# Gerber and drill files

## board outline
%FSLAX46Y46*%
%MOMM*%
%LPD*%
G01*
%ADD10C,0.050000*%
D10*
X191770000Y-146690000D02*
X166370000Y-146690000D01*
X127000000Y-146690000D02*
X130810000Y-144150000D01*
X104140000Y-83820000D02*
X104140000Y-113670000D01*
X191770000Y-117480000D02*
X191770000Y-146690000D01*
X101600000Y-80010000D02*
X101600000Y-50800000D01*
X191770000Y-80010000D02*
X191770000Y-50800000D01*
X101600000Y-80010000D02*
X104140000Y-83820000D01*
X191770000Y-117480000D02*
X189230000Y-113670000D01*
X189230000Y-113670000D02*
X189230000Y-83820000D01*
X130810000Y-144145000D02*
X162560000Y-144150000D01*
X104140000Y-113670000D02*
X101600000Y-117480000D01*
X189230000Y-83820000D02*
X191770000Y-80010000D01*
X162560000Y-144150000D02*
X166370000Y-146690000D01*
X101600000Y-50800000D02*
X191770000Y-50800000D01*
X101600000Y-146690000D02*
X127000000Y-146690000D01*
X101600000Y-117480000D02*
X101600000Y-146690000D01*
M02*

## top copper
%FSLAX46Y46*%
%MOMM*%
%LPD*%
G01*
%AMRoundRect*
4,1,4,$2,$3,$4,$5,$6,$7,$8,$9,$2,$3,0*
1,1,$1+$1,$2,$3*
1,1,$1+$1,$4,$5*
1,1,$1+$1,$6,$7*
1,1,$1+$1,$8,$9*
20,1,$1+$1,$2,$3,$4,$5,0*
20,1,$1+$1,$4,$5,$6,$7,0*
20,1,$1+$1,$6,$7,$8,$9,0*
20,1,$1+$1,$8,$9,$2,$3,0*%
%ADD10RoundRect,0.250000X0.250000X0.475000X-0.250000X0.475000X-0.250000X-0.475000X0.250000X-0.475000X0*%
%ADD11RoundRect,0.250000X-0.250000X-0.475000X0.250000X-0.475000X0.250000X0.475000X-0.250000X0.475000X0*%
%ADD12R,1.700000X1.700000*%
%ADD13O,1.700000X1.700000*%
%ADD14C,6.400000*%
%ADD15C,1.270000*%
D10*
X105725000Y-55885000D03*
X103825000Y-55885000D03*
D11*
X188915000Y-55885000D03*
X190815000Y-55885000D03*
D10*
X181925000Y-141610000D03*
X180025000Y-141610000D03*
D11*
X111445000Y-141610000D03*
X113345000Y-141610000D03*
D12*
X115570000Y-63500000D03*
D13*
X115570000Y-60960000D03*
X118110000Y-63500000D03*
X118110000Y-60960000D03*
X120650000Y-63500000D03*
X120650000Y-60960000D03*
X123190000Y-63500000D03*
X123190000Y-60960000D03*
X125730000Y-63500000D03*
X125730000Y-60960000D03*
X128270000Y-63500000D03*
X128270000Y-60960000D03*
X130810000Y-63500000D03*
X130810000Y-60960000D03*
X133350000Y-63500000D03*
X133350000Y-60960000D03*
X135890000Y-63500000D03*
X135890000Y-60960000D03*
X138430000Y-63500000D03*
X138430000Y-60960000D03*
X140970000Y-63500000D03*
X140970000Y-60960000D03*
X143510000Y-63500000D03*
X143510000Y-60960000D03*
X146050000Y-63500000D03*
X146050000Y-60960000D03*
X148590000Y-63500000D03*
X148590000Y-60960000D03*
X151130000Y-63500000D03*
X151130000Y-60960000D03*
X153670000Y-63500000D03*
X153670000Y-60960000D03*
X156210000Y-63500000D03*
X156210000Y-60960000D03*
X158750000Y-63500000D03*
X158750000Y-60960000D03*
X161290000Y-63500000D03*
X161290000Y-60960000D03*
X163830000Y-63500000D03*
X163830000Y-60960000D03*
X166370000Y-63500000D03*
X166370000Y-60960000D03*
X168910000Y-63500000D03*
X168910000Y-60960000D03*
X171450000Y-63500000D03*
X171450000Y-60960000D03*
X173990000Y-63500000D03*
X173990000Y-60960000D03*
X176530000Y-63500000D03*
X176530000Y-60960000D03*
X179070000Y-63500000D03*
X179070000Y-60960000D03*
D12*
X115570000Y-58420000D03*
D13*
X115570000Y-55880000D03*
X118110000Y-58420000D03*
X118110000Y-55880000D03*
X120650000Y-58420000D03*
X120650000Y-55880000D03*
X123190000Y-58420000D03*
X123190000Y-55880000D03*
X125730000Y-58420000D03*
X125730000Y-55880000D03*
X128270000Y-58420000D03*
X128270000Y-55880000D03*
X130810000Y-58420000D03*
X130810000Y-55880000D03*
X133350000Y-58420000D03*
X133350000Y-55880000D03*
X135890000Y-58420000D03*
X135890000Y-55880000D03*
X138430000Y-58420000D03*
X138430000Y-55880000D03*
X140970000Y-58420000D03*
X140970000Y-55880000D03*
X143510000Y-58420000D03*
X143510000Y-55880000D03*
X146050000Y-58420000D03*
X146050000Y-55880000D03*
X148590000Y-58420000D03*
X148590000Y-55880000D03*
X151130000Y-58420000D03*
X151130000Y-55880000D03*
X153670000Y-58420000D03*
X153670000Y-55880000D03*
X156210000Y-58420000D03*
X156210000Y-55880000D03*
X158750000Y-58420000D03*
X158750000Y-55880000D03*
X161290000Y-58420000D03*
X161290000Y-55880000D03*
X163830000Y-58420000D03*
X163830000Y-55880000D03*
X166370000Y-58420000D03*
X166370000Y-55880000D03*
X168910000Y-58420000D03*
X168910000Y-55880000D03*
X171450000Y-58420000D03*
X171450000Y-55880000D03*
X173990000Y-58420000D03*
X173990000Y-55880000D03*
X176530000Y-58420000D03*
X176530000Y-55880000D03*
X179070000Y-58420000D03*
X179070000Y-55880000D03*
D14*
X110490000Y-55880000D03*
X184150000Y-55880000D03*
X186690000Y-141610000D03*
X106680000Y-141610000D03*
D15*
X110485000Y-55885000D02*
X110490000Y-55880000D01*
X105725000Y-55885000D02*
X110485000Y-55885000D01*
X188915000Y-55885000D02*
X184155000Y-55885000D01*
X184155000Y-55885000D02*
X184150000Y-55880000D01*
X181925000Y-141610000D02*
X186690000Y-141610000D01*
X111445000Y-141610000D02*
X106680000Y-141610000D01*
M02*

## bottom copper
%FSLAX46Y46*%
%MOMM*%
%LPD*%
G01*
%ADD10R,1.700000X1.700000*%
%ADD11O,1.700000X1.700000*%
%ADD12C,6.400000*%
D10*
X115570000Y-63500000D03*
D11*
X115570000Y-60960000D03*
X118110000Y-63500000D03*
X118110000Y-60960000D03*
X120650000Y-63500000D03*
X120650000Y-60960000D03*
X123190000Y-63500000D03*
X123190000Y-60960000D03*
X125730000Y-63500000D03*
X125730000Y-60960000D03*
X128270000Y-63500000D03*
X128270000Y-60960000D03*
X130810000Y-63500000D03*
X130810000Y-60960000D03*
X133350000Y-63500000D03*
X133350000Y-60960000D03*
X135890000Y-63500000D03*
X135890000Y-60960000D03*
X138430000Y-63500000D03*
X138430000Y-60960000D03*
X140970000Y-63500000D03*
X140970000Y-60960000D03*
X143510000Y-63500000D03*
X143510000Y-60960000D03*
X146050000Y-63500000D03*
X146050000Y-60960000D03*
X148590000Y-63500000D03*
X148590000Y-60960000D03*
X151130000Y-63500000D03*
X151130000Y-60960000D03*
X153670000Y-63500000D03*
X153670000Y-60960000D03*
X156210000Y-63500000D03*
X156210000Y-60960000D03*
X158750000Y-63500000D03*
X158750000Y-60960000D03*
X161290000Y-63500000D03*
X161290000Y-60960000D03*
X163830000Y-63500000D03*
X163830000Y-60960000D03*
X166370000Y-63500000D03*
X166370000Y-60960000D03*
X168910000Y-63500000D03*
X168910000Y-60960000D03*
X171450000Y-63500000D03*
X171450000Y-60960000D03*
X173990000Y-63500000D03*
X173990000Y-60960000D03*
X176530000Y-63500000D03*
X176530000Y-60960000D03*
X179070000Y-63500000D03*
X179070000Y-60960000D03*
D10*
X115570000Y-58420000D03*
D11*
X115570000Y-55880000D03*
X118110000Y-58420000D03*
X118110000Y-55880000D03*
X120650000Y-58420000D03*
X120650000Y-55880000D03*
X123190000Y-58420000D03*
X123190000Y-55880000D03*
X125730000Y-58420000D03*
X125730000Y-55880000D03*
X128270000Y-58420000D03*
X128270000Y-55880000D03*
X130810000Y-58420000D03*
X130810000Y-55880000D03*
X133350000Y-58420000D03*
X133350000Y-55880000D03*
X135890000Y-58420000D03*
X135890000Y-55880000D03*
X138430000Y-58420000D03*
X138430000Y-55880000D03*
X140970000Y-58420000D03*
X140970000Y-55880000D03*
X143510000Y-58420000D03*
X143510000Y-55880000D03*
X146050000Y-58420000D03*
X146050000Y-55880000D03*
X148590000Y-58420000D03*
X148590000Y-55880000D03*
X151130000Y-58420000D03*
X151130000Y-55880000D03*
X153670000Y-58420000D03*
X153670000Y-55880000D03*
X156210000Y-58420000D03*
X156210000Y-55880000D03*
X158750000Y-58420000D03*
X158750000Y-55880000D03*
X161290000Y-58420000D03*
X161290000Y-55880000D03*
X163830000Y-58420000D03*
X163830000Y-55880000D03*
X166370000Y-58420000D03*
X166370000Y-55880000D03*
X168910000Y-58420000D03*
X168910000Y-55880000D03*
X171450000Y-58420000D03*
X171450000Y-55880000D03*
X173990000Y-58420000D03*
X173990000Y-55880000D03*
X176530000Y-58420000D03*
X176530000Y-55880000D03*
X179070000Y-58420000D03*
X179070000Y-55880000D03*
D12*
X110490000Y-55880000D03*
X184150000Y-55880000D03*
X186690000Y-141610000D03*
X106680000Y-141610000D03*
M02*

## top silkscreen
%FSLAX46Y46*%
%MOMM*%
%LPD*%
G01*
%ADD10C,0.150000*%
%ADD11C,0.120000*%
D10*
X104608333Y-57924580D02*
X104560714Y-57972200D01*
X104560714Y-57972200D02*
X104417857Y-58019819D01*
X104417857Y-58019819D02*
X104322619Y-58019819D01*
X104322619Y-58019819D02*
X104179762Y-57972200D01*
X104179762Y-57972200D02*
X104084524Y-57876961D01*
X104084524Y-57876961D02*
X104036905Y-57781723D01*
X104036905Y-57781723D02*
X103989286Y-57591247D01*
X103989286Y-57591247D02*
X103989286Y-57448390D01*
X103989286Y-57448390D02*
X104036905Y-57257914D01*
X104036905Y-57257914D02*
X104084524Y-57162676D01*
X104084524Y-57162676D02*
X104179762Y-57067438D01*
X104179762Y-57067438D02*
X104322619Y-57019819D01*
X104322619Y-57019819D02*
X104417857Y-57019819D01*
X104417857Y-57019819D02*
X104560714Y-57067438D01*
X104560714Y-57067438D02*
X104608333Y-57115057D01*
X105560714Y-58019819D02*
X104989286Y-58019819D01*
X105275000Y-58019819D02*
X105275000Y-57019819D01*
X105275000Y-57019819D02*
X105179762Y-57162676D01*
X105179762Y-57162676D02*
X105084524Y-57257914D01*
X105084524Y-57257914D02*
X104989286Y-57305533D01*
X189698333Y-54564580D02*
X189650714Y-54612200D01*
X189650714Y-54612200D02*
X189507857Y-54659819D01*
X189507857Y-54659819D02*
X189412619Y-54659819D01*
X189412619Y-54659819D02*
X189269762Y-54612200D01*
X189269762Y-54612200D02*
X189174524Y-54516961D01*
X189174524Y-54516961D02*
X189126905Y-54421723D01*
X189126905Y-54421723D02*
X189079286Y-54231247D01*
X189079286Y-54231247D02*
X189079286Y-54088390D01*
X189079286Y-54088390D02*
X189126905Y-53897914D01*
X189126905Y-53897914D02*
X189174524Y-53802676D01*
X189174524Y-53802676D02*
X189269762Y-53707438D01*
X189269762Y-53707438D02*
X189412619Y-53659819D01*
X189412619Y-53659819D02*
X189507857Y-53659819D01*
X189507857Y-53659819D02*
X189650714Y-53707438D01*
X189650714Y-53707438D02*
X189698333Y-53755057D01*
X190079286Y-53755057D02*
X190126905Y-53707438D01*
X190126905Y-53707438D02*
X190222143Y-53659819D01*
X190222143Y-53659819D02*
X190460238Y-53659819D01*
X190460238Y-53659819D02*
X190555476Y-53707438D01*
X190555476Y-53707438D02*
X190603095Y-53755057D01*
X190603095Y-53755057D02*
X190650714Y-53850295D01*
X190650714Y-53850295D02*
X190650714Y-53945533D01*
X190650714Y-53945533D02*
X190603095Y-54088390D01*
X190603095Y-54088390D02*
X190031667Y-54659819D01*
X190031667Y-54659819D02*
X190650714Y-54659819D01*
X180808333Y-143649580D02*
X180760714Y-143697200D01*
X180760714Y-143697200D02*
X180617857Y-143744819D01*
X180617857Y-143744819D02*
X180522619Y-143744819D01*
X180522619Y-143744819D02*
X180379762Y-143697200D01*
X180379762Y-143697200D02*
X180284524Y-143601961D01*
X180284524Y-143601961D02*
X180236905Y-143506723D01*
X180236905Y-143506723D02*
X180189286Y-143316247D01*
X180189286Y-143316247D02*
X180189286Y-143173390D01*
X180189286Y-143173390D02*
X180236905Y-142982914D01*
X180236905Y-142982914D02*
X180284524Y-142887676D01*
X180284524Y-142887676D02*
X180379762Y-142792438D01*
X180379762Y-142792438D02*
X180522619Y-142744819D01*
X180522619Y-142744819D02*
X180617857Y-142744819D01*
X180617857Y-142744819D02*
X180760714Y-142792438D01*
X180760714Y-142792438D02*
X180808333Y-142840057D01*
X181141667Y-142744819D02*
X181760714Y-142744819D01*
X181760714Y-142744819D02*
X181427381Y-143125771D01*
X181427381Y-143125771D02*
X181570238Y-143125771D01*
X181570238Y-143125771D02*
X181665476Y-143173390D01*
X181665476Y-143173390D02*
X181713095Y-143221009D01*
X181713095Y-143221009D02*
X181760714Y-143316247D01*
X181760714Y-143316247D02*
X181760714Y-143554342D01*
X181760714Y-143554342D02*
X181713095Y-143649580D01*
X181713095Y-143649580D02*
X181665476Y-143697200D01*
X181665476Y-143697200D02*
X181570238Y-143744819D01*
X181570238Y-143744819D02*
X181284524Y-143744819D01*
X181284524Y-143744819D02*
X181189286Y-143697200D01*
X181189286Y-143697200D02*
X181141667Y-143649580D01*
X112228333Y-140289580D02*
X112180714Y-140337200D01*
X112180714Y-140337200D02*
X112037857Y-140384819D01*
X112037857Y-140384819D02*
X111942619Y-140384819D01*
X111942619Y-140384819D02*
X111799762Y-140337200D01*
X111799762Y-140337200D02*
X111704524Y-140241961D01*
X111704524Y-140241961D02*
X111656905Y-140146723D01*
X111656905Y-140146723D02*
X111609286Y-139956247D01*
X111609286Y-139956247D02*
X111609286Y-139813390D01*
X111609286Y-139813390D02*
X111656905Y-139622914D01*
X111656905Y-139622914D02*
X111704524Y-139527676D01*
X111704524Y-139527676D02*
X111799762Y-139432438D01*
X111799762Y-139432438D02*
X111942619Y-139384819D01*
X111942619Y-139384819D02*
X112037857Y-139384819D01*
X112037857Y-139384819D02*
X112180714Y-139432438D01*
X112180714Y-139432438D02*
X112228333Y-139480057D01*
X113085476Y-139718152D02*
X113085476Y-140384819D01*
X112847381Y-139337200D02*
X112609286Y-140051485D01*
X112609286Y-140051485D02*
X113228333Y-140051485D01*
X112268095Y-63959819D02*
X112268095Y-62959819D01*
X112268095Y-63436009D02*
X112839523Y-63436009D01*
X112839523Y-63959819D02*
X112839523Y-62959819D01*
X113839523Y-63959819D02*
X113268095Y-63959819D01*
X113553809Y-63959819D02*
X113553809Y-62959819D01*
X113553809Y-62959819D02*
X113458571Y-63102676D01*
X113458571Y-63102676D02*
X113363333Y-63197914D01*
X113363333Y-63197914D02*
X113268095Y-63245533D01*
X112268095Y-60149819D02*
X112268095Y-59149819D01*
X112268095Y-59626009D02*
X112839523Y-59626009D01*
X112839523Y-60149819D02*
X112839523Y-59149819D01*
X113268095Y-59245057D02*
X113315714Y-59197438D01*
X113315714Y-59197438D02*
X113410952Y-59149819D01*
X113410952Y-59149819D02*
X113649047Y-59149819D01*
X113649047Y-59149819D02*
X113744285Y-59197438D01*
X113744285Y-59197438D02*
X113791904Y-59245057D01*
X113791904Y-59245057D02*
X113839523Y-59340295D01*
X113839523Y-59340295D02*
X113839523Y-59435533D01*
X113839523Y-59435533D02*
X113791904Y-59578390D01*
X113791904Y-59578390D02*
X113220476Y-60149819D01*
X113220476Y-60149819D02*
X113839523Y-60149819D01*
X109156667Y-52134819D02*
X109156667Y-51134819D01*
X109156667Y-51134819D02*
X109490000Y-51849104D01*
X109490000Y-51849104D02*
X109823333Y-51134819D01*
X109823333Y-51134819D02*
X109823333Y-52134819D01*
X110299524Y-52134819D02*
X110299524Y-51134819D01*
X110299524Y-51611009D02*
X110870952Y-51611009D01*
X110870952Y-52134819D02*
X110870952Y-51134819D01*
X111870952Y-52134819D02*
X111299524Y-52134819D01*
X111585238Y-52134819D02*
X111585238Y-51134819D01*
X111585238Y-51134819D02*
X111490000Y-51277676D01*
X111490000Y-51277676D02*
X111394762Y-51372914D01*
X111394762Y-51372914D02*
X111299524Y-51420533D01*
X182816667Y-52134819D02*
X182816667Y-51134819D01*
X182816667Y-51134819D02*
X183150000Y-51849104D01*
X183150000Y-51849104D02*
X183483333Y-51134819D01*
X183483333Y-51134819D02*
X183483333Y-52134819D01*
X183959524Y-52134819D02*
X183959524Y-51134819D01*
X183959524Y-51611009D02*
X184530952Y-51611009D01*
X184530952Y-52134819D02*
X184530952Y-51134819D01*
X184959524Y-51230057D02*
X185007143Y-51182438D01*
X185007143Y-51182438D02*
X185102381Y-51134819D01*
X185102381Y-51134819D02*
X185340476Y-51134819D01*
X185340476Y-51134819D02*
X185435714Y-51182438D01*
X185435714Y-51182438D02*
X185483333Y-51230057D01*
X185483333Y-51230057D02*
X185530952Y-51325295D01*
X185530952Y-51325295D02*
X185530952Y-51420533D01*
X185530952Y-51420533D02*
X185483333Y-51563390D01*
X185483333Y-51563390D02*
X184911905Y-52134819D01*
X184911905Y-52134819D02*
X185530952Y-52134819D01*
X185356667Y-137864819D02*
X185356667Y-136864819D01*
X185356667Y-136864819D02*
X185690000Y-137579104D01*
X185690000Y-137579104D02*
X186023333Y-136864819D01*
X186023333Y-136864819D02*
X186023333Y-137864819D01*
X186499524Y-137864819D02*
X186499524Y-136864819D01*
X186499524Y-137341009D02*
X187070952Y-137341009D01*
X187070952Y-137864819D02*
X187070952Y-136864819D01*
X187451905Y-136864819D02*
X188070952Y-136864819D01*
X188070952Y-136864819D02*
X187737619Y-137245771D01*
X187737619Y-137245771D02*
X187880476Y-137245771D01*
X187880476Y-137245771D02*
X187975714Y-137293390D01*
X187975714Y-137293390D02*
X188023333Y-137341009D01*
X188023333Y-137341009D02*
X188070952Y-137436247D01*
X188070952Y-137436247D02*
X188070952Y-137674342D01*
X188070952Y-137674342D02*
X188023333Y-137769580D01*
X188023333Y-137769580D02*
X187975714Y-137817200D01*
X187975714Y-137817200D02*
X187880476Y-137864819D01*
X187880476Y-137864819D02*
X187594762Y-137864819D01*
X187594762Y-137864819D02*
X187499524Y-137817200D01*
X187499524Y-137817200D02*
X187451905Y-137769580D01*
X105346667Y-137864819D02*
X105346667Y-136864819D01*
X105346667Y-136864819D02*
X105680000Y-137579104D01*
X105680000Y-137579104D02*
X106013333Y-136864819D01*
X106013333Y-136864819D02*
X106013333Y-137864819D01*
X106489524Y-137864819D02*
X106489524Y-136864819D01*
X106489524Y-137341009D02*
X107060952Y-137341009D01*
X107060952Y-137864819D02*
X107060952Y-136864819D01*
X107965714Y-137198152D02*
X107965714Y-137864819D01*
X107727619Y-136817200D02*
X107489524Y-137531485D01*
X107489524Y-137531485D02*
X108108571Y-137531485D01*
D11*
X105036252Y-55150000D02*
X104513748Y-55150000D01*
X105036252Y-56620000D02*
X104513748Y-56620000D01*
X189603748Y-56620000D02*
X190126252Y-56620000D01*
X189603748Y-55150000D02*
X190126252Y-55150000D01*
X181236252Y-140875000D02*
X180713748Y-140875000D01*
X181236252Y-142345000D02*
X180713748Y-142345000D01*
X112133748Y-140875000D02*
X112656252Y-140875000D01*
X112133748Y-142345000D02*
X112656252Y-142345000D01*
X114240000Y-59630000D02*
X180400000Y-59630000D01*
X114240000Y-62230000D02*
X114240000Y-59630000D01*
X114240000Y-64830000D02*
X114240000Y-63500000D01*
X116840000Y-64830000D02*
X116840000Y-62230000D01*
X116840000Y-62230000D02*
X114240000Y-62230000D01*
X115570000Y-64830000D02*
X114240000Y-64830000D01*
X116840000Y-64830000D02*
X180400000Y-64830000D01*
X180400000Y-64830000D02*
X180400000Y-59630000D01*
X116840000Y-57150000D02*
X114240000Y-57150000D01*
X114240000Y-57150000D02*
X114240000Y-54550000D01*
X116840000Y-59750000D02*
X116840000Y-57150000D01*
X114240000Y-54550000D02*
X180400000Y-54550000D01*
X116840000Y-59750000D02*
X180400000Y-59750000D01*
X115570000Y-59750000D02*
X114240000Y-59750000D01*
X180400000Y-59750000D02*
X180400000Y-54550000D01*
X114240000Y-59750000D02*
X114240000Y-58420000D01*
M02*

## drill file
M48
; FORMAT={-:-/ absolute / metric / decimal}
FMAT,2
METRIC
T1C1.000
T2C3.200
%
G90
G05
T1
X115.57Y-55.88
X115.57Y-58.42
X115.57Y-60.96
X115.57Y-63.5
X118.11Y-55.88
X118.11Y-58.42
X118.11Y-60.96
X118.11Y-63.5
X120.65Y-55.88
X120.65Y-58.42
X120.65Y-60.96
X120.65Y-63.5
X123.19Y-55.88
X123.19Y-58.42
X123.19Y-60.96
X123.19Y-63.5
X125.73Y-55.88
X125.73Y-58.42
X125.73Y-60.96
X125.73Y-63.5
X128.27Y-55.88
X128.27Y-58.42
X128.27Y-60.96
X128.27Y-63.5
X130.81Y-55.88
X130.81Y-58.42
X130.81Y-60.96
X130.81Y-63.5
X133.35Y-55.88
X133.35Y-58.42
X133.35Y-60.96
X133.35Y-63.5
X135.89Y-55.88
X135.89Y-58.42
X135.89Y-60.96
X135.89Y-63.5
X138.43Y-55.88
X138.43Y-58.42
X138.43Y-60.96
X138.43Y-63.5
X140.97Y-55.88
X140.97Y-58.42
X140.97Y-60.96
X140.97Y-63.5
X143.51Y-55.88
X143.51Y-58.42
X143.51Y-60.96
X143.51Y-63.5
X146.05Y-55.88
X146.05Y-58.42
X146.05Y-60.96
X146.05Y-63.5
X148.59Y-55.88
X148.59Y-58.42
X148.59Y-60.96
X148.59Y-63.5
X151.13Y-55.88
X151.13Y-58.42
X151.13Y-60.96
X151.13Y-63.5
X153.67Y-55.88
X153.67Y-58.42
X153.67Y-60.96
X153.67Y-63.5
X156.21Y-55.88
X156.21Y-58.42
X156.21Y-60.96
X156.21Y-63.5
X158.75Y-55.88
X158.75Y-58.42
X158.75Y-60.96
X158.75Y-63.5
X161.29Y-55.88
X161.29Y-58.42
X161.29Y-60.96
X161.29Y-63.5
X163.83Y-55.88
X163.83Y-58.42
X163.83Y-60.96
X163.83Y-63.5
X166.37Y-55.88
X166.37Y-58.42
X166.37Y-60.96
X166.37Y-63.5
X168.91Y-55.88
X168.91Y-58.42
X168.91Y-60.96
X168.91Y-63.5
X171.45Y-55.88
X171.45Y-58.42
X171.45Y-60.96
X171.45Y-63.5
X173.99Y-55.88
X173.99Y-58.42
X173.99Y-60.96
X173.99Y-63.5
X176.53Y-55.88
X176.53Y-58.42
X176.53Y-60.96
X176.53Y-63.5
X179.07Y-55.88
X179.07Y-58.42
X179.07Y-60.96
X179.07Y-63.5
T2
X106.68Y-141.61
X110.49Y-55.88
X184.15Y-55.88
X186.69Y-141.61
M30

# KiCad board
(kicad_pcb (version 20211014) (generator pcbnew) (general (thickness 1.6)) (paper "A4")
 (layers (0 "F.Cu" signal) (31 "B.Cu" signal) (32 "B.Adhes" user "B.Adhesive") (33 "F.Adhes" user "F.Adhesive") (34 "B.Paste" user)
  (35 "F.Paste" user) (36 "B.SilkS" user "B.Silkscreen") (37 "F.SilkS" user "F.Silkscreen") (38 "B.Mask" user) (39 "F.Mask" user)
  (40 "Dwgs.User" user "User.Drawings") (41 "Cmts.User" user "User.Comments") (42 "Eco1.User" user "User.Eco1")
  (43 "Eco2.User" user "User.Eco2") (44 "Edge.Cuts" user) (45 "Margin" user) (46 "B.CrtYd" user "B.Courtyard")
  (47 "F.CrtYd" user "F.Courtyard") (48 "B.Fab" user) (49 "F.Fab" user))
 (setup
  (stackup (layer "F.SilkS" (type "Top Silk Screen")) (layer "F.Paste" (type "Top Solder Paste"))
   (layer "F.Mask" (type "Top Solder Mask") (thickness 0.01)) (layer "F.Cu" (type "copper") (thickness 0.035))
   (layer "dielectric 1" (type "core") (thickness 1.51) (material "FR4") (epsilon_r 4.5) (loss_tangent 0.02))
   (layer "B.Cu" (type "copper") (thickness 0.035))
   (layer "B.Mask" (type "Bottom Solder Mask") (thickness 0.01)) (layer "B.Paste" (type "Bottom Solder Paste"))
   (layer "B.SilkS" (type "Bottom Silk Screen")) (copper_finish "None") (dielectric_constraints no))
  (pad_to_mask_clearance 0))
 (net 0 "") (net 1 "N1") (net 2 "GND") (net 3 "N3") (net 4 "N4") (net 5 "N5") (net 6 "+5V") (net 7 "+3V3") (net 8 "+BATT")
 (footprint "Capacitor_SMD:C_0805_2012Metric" (layer "F.Cu") (at 104.775 55.885 180)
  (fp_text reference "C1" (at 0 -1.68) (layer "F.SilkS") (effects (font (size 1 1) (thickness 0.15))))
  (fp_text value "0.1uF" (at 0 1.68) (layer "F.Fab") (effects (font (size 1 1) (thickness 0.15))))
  (fp_line (start -0.261252 0.735) (end 0.261252 0.735) (layer "F.SilkS") (width 0.12))
  (fp_line (start -0.261252 -0.735) (end 0.261252 -0.735) (layer "F.SilkS") (width 0.12))
  (pad "1" smd roundrect locked (at -0.95 0 180) (size 1 1.45) (layers "F.Cu" "F.Paste" "F.Mask") (roundrect_rratio 0.25) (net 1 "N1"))
  (pad "2" smd roundrect locked (at 0.95 0 180) (size 1 1.45) (layers "F.Cu" "F.Paste" "F.Mask") (roundrect_rratio 0.25) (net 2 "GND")))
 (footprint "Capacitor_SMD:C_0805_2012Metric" (layer "F.Cu") (at 189.865 55.885)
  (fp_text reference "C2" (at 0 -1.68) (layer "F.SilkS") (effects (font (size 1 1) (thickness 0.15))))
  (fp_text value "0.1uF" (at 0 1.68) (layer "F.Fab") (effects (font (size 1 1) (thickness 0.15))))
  (fp_line (start -0.261252 0.735) (end 0.261252 0.735) (layer "F.SilkS") (width 0.12))
  (fp_line (start -0.261252 -0.735) (end 0.261252 -0.735) (layer "F.SilkS") (width 0.12))
  (pad "1" smd roundrect locked (at -0.95 0) (size 1 1.45) (layers "F.Cu" "F.Paste" "F.Mask") (roundrect_rratio 0.25) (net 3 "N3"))
  (pad "2" smd roundrect locked (at 0.95 0) (size 1 1.45) (layers "F.Cu" "F.Paste" "F.Mask") (roundrect_rratio 0.25) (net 2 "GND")))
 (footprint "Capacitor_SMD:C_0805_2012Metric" (layer "F.Cu") (at 180.975 141.61 180)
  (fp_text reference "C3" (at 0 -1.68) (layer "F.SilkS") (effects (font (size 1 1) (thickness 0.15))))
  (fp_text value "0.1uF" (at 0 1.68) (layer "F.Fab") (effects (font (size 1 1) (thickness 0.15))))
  (fp_line (start -0.261252 0.735) (end 0.261252 0.735) (layer "F.SilkS") (width 0.12))
  (fp_line (start -0.261252 -0.735) (end 0.261252 -0.735) (layer "F.SilkS") (width 0.12))
  (pad "1" smd roundrect locked (at -0.95 0 180) (size 1 1.45) (layers "F.Cu" "F.Paste" "F.Mask") (roundrect_rratio 0.25) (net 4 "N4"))
  (pad "2" smd roundrect locked (at 0.95 0 180) (size 1 1.45) (layers "F.Cu" "F.Paste" "F.Mask") (roundrect_rratio 0.25) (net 2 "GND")))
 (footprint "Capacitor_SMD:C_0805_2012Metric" (layer "F.Cu") (at 112.395 141.61)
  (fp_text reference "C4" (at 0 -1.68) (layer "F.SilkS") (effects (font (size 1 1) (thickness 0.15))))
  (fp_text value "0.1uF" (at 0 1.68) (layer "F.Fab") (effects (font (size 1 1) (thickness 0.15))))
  (fp_line (start -0.261252 -0.735) (end 0.261252 -0.735) (layer "F.SilkS") (width 0.12))
  (fp_line (start -0.261252 0.735) (end 0.261252 0.735) (layer "F.SilkS") (width 0.12))
  (pad "1" smd roundrect locked (at -0.95 0) (size 1 1.45) (layers "F.Cu" "F.Paste" "F.Mask") (roundrect_rratio 0.25) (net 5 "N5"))
  (pad "2" smd roundrect locked (at 0.95 0) (size 1 1.45) (layers "F.Cu" "F.Paste" "F.Mask") (roundrect_rratio 0.25) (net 2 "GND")))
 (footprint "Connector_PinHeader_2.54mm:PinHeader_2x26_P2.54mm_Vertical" (layer "F.Cu") (at 115.57 63.5 90)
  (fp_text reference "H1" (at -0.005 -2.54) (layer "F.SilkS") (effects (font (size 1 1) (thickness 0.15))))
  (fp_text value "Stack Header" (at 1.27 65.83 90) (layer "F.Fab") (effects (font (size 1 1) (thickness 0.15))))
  (fp_line (start 3.87 -1.33) (end 3.87 64.83) (layer "F.SilkS") (width 0.12))
  (fp_line (start 1.27 -1.33) (end 3.87 -1.33) (layer "F.SilkS") (width 0.12))
  (fp_line (start -1.33 -1.33) (end 0 -1.33) (layer "F.SilkS") (width 0.12))
  (fp_line (start -1.33 1.27) (end 1.27 1.27) (layer "F.SilkS") (width 0.12))
  (fp_line (start 1.27 1.27) (end 1.27 -1.33) (layer "F.SilkS") (width 0.12))
  (fp_line (start -1.33 0) (end -1.33 -1.33) (layer "F.SilkS") (width 0.12))
  (fp_line (start -1.33 1.27) (end -1.33 64.83) (layer "F.SilkS") (width 0.12))
  (fp_line (start -1.33 64.83) (end 3.87 64.83) (layer "F.SilkS") (width 0.12))
  (pad "1" thru_hole rect locked (at 0 0 90) (size 1.7 1.7) (drill 1) (layers *.Cu *.Mask))
  (pad "2" thru_hole oval locked (at 2.54 0 90) (size 1.7 1.7) (drill 1) (layers *.Cu *.Mask))
  (pad "3" thru_hole oval locked (at 0 2.54 90) (size 1.7 1.7) (drill 1) (layers *.Cu *.Mask))
  (pad "4" thru_hole oval locked (at 2.54 2.54 90) (size 1.7 1.7) (drill 1) (layers *.Cu *.Mask))
  (pad "5" thru_hole oval locked (at 0 5.08 90) (size 1.7 1.7) (drill 1) (layers *.Cu *.Mask))
  (pad "6" thru_hole oval locked (at 2.54 5.08 90) (size 1.7 1.7) (drill 1) (layers *.Cu *.Mask))
  (pad "7" thru_hole oval locked (at 0 7.62 90) (size 1.7 1.7) (drill 1) (layers *.Cu *.Mask))
  (pad "8" thru_hole oval locked (at 2.54 7.62 90) (size 1.7 1.7) (drill 1) (layers *.Cu *.Mask))
  (pad "9" thru_hole oval locked (at 0 10.16 90) (size 1.7 1.7) (drill 1) (layers *.Cu *.Mask))
  (pad "10" thru_hole oval locked (at 2.54 10.16 90) (size 1.7 1.7) (drill 1) (layers *.Cu *.Mask))
  (pad "11" thru_hole oval locked (at 0 12.7 90) (size 1.7 1.7) (drill 1) (layers *.Cu *.Mask))
  (pad "12" thru_hole oval locked (at 2.54 12.7 90) (size 1.7 1.7) (drill 1) (layers *.Cu *.Mask))
  (pad "13" thru_hole oval locked (at 0 15.24 90) (size 1.7 1.7) (drill 1) (layers *.Cu *.Mask))
  (pad "14" thru_hole oval locked (at 2.54 15.24 90) (size 1.7 1.7) (drill 1) (layers *.Cu *.Mask))
  (pad "15" thru_hole oval locked (at 0 17.78 90) (size 1.7 1.7) (drill 1) (layers *.Cu *.Mask))
  (pad "16" thru_hole oval locked (at 2.54 17.78 90) (size 1.7 1.7) (drill 1) (layers *.Cu *.Mask))
  (pad "17" thru_hole oval locked (at 0 20.32 90) (size 1.7 1.7) (drill 1) (layers *.Cu *.Mask))
  (pad "18" thru_hole oval locked (at 2.54 20.32 90) (size 1.7 1.7) (drill 1) (layers *.Cu *.Mask))
  (pad "19" thru_hole oval locked (at 0 22.86 90) (size 1.7 1.7) (drill 1) (layers *.Cu *.Mask))
  (pad "20" thru_hole oval locked (at 2.54 22.86 90) (size 1.7 1.7) (drill 1) (layers *.Cu *.Mask))
  (pad "21" thru_hole oval locked (at 0 25.4 90) (size 1.7 1.7) (drill 1) (layers *.Cu *.Mask))
  (pad "22" thru_hole oval locked (at 2.54 25.4 90) (size 1.7 1.7) (drill 1) (layers *.Cu *.Mask))
  (pad "23" thru_hole oval locked (at 0 27.94 90) (size 1.7 1.7) (drill 1) (layers *.Cu *.Mask))
  (pad "24" thru_hole oval locked (at 2.54 27.94 90) (size 1.7 1.7) (drill 1) (layers *.Cu *.Mask))
  (pad "25" thru_hole oval locked (at 0 30.48 90) (size 1.7 1.7) (drill 1) (layers *.Cu *.Mask))
  (pad "26" thru_hole oval locked (at 2.54 30.48 90) (size 1.7 1.7) (drill 1) (layers *.Cu *.Mask))
  (pad "27" thru_hole oval locked (at 0 33.02 90) (size 1.7 1.7) (drill 1) (layers *.Cu *.Mask))
  (pad "28" thru_hole oval locked (at 2.54 33.02 90) (size 1.7 1.7) (drill 1) (layers *.Cu *.Mask))
  (pad "29" thru_hole oval locked (at 0 35.56 90) (size 1.7 1.7) (drill 1) (layers *.Cu *.Mask))
  (pad "30" thru_hole oval locked (at 2.54 35.56 90) (size 1.7 1.7) (drill 1) (layers *.Cu *.Mask))
  (pad "31" thru_hole oval locked (at 0 38.1 90) (size 1.7 1.7) (drill 1) (layers *.Cu *.Mask))
  (pad "32" thru_hole oval locked (at 2.54 38.1 90) (size 1.7 1.7) (drill 1) (layers *.Cu *.Mask))
  (pad "33" thru_hole oval locked (at 0 40.64 90) (size 1.7 1.7) (drill 1) (layers *.Cu *.Mask))
  (pad "34" thru_hole oval locked (at 2.54 40.64 90) (size 1.7 1.7) (drill 1) (layers *.Cu *.Mask))
  (pad "35" thru_hole oval locked (at 0 43.18 90) (size 1.7 1.7) (drill 1) (layers *.Cu *.Mask))
  (pad "36" thru_hole oval locked (at 2.54 43.18 90) (size 1.7 1.7) (drill 1) (layers *.Cu *.Mask))
  (pad "37" thru_hole oval locked (at 0 45.72 90) (size 1.7 1.7) (drill 1) (layers *.Cu *.Mask))
  (pad "38" thru_hole oval locked (at 2.54 45.72 90) (size 1.7 1.7) (drill 1) (layers *.Cu *.Mask))
  (pad "39" thru_hole oval locked (at 0 48.26 90) (size 1.7 1.7) (drill 1) (layers *.Cu *.Mask))
  (pad "40" thru_hole oval locked (at 2.54 48.26 90) (size 1.7 1.7) (drill 1) (layers *.Cu *.Mask))
  (pad "41" thru_hole oval locked (at 0 50.8 90) (size 1.7 1.7) (drill 1) (layers *.Cu *.Mask))
  (pad "42" thru_hole oval locked (at 2.54 50.8 90) (size 1.7 1.7) (drill 1) (layers *.Cu *.Mask))
  (pad "43" thru_hole oval locked (at 0 53.34 90) (size 1.7 1.7) (drill 1) (layers *.Cu *.Mask))
  (pad "44" thru_hole oval locked (at 2.54 53.34 90) (size 1.7 1.7) (drill 1) (layers *.Cu *.Mask))
  (pad "45" thru_hole oval locked (at 0 55.88 90) (size 1.7 1.7) (drill 1) (layers *.Cu *.Mask))
  (pad "46" thru_hole oval locked (at 2.54 55.88 90) (size 1.7 1.7) (drill 1) (layers *.Cu *.Mask))
  (pad "47" thru_hole oval locked (at 0 58.42 90) (size 1.7 1.7) (drill 1) (layers *.Cu *.Mask))
  (pad "48" thru_hole oval locked (at 2.54 58.42 90) (size 1.7 1.7) (drill 1) (layers *.Cu *.Mask))
  (pad "49" thru_hole oval locked (at 0 60.96 90) (size 1.7 1.7) (drill 1) (layers *.Cu *.Mask))
  (pad "50" thru_hole oval locked (at 2.54 60.96 90) (size 1.7 1.7) (drill 1) (layers *.Cu *.Mask))
  (pad "51" thru_hole oval locked (at 0 63.5 90) (size 1.7 1.7) (drill 1) (layers *.Cu *.Mask))
  (pad "52" thru_hole oval locked (at 2.54 63.5 90) (size 1.7 1.7) (drill 1) (layers *.Cu *.Mask)))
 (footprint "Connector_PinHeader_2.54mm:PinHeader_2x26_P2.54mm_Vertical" (layer "F.Cu") (at 115.57 58.42 90)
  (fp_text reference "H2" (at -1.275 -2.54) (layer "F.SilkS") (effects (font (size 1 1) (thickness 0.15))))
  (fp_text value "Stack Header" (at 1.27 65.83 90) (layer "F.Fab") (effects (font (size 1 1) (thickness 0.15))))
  (fp_line (start 1.27 1.27) (end 1.27 -1.33) (layer "F.SilkS") (width 0.12))
  (fp_line (start 1.27 -1.33) (end 3.87 -1.33) (layer "F.SilkS") (width 0.12))
  (fp_line (start -1.33 1.27) (end 1.27 1.27) (layer "F.SilkS") (width 0.12))
  (fp_line (start 3.87 -1.33) (end 3.87 64.83) (layer "F.SilkS") (width 0.12))
  (fp_line (start -1.33 1.27) (end -1.33 64.83) (layer "F.SilkS") (width 0.12))
  (fp_line (start -1.33 0) (end -1.33 -1.33) (layer "F.SilkS") (width 0.12))
  (fp_line (start -1.33 64.83) (end 3.87 64.83) (layer "F.SilkS") (width 0.12))
  (fp_line (start -1.33 -1.33) (end 0 -1.33) (layer "F.SilkS") (width 0.12))
  (pad "1" thru_hole rect locked (at 0 0 90) (size 1.7 1.7) (drill 1) (layers *.Cu *.Mask))
  (pad "2" thru_hole oval locked (at 2.54 0 90) (size 1.7 1.7) (drill 1) (layers *.Cu *.Mask))
  (pad "3" thru_hole oval locked (at 0 2.54 90) (size 1.7 1.7) (drill 1) (layers *.Cu *.Mask))
  (pad "4" thru_hole oval locked (at 2.54 2.54 90) (size 1.7 1.7) (drill 1) (layers *.Cu *.Mask))
  (pad "5" thru_hole oval locked (at 0 5.08 90) (size 1.7 1.7) (drill 1) (layers *.Cu *.Mask))
  (pad "6" thru_hole oval locked (at 2.54 5.08 90) (size 1.7 1.7) (drill 1) (layers *.Cu *.Mask))
  (pad "7" thru_hole oval locked (at 0 7.62 90) (size 1.7 1.7) (drill 1) (layers *.Cu *.Mask))
  (pad "8" thru_hole oval locked (at 2.54 7.62 90) (size 1.7 1.7) (drill 1) (layers *.Cu *.Mask))
  (pad "9" thru_hole oval locked (at 0 10.16 90) (size 1.7 1.7) (drill 1) (layers *.Cu *.Mask))
  (pad "10" thru_hole oval locked (at 2.54 10.16 90) (size 1.7 1.7) (drill 1) (layers *.Cu *.Mask))
  (pad "11" thru_hole oval locked (at 0 12.7 90) (size 1.7 1.7) (drill 1) (layers *.Cu *.Mask))
  (pad "12" thru_hole oval locked (at 2.54 12.7 90) (size 1.7 1.7) (drill 1) (layers *.Cu *.Mask))
  (pad "13" thru_hole oval locked (at 0 15.24 90) (size 1.7 1.7) (drill 1) (layers *.Cu *.Mask))
  (pad "14" thru_hole oval locked (at 2.54 15.24 90) (size 1.7 1.7) (drill 1) (layers *.Cu *.Mask))
  (pad "15" thru_hole oval locked (at 0 17.78 90) (size 1.7 1.7) (drill 1) (layers *.Cu *.Mask))
  (pad "16" thru_hole oval locked (at 2.54 17.78 90) (size 1.7 1.7) (drill 1) (layers *.Cu *.Mask))
  (pad "17" thru_hole oval locked (at 0 20.32 90) (size 1.7 1.7) (drill 1) (layers *.Cu *.Mask))
  (pad "18" thru_hole oval locked (at 2.54 20.32 90) (size 1.7 1.7) (drill 1) (layers *.Cu *.Mask))
  (pad "19" thru_hole oval locked (at 0 22.86 90) (size 1.7 1.7) (drill 1) (layers *.Cu *.Mask))
  (pad "20" thru_hole oval locked (at 2.54 22.86 90) (size 1.7 1.7) (drill 1) (layers *.Cu *.Mask))
  (pad "21" thru_hole oval locked (at 0 25.4 90) (size 1.7 1.7) (drill 1) (layers *.Cu *.Mask))
  (pad "22" thru_hole oval locked (at 2.54 25.4 90) (size 1.7 1.7) (drill 1) (layers *.Cu *.Mask))
  (pad "23" thru_hole oval locked (at 0 27.94 90) (size 1.7 1.7) (drill 1) (layers *.Cu *.Mask))
  (pad "24" thru_hole oval locked (at 2.54 27.94 90) (size 1.7 1.7) (drill 1) (layers *.Cu *.Mask))
  (pad "25" thru_hole oval locked (at 0 30.48 90) (size 1.7 1.7) (drill 1) (layers *.Cu *.Mask) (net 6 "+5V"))
  (pad "26" thru_hole oval locked (at 2.54 30.48 90) (size 1.7 1.7) (drill 1) (layers *.Cu *.Mask) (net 6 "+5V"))
  (pad "27" thru_hole oval locked (at 0 33.02 90) (size 1.7 1.7) (drill 1) (layers *.Cu *.Mask) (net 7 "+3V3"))
  (pad "28" thru_hole oval locked (at 2.54 33.02 90) (size 1.7 1.7) (drill 1) (layers *.Cu *.Mask) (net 7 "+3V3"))
  (pad "29" thru_hole oval locked (at 0 35.56 90) (size 1.7 1.7) (drill 1) (layers *.Cu *.Mask) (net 2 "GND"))
  (pad "30" thru_hole oval locked (at 2.54 35.56 90) (size 1.7 1.7) (drill 1) (layers *.Cu *.Mask) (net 2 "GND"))
  (pad "31" thru_hole oval locked (at 0 38.1 90) (size 1.7 1.7) (drill 1) (layers *.Cu *.Mask))
  (pad "32" thru_hole oval locked (at 2.54 38.1 90) (size 1.7 1.7) (drill 1) (layers *.Cu *.Mask) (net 2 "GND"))
  (pad "33" thru_hole oval locked (at 0 40.64 90) (size 1.7 1.7) (drill 1) (layers *.Cu *.Mask))
  (pad "34" thru_hole oval locked (at 2.54 40.64 90) (size 1.7 1.7) (drill 1) (layers *.Cu *.Mask))
  (pad "35" thru_hole oval locked (at 0 43.18 90) (size 1.7 1.7) (drill 1) (layers *.Cu *.Mask))
  (pad "36" thru_hole oval locked (at 2.54 43.18 90) (size 1.7 1.7) (drill 1) (layers *.Cu *.Mask))
  (pad "37" thru_hole oval locked (at 0 45.72 90) (size 1.7 1.7) (drill 1) (layers *.Cu *.Mask))
  (pad "38" thru_hole oval locked (at 2.54 45.72 90) (size 1.7 1.7) (drill 1) (layers *.Cu *.Mask))
  (pad "39" thru_hole oval locked (at 0 48.26 90) (size 1.7 1.7) (drill 1) (layers *.Cu *.Mask))
  (pad "40" thru_hole oval locked (at 2.54 48.26 90) (size 1.7 1.7) (drill 1) (layers *.Cu *.Mask))
  (pad "41" thru_hole oval locked (at 0 50.8 90) (size 1.7 1.7) (drill 1) (layers *.Cu *.Mask))
  (pad "42" thru_hole oval locked (at 2.54 50.8 90) (size 1.7 1.7) (drill 1) (layers *.Cu *.Mask))
  (pad "43" thru_hole oval locked (at 0 53.34 90) (size 1.7 1.7) (drill 1) (layers *.Cu *.Mask))
  (pad "44" thru_hole oval locked (at 2.54 53.34 90) (size 1.7 1.7) (drill 1) (layers *.Cu *.Mask))
  (pad "45" thru_hole oval locked (at 0 55.88 90) (size 1.7 1.7) (drill 1) (layers *.Cu *.Mask) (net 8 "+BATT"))
  (pad "46" thru_hole oval locked (at 2.54 55.88 90) (size 1.7 1.7) (drill 1) (layers *.Cu *.Mask) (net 8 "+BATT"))
  (pad "47" thru_hole oval locked (at 0 58.42 90) (size 1.7 1.7) (drill 1) (layers *.Cu *.Mask))
  (pad "48" thru_hole oval locked (at 2.54 58.42 90) (size 1.7 1.7) (drill 1) (layers *.Cu *.Mask))
  (pad "49" thru_hole oval locked (at 0 60.96 90) (size 1.7 1.7) (drill 1) (layers *.Cu *.Mask))
  (pad "50" thru_hole oval locked (at 2.54 60.96 90) (size 1.7 1.7) (drill 1) (layers *.Cu *.Mask))
  (pad "51" thru_hole oval locked (at 0 63.5 90) (size 1.7 1.7) (drill 1) (layers *.Cu *.Mask))
  (pad "52" thru_hole oval locked (at 2.54 63.5 90) (size 1.7 1.7) (drill 1) (layers *.Cu *.Mask)))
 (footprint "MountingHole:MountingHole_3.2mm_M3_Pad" (layer "F.Cu") (at 110.49 55.88)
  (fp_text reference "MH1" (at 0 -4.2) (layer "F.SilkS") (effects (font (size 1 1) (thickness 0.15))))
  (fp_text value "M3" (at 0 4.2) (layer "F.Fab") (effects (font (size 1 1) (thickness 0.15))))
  (pad "1" thru_hole circle locked (at 0 0) (size 6.4 6.4) (drill 3.2) (layers *.Cu *.Mask) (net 1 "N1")))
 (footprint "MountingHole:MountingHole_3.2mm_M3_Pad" (layer "F.Cu") (at 184.15 55.88)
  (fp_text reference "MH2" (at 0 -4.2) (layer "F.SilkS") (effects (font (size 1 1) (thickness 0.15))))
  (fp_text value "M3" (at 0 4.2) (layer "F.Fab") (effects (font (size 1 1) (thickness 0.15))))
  (pad "1" thru_hole circle locked (at 0 0) (size 6.4 6.4) (drill 3.2) (layers *.Cu *.Mask) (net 3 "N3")))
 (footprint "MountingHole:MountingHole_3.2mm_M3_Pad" (layer "F.Cu") (at 186.69 141.61)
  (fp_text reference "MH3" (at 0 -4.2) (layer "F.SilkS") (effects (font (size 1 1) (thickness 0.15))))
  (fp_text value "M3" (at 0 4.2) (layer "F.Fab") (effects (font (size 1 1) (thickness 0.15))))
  (pad "1" thru_hole circle locked (at 0 0) (size 6.4 6.4) (drill 3.2) (layers *.Cu *.Mask) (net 4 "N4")))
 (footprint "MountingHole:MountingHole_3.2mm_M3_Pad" (layer "F.Cu") (at 106.68 141.61)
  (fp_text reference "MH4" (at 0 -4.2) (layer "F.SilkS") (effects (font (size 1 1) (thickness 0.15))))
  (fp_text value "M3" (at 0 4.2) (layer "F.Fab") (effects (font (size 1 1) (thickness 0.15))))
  (pad "1" thru_hole circle locked (at 0 0) (size 6.4 6.4) (drill 3.2) (layers *.Cu *.Mask) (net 5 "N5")))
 (gr_line (start 191.77 146.69) (end 166.37 146.69) (layer "Edge.Cuts") (width 0.05))
 (gr_line (start 127 146.69) (end 130.81 144.15) (layer "Edge.Cuts") (width 0.05))
 (gr_line (start 104.14 83.82) (end 104.14 113.67) (layer "Edge.Cuts") (width 0.05))
 (gr_line (start 191.77 117.48) (end 191.77 146.69) (layer "Edge.Cuts") (width 0.05))
 (gr_line (start 101.6 80.01) (end 101.6 50.8) (layer "Edge.Cuts") (width 0.05))
 (gr_line (start 191.77 80.01) (end 191.77 50.8) (layer "Edge.Cuts") (width 0.05))
 (gr_line (start 101.6 80.01) (end 104.14 83.82) (layer "Edge.Cuts") (width 0.05))
 (gr_line (start 191.77 117.48) (end 189.23 113.67) (layer "Edge.Cuts") (width 0.05))
 (gr_line (start 189.23 113.67) (end 189.23 83.82) (layer "Edge.Cuts") (width 0.05))
 (gr_line (start 130.81 144.145) (end 162.56 144.15) (layer "Edge.Cuts") (width 0.05))
 (gr_line (start 104.14 113.67) (end 101.6 117.48) (layer "Edge.Cuts") (width 0.05))
 (gr_line (start 189.23 83.82) (end 191.77 80.01) (layer "Edge.Cuts") (width 0.05))
 (gr_line (start 162.56 144.15) (end 166.37 146.69) (layer "Edge.Cuts") (width 0.05))
 (gr_line (start 101.6 50.8) (end 191.77 50.8) (layer "Edge.Cuts") (width 0.05))
 (gr_line (start 101.6 146.69) (end 127 146.69) (layer "Edge.Cuts") (width 0.05))
 (gr_line (start 101.6 117.48) (end 101.6 146.69) (layer "Edge.Cuts") (width 0.05))
 (segment (start 110.485 55.885) (end 110.49 55.88) (width 1.27) (layer "F.Cu") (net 1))
 (segment (start 105.725 55.885) (end 110.485 55.885) (width 1.27) (layer "F.Cu") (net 1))
 (segment (start 188.915 55.885) (end 184.155 55.885) (width 1.27) (layer "F.Cu") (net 3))
 (segment (start 184.155 55.885) (end 184.15 55.88) (width 1.27) (layer "F.Cu") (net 3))
 (segment (start 181.925 141.61) (end 186.69 141.61) (width 1.27) (layer "F.Cu") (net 4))
 (segment (start 111.445 141.61) (end 106.68 141.61) (width 1.27) (layer "F.Cu") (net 5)))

